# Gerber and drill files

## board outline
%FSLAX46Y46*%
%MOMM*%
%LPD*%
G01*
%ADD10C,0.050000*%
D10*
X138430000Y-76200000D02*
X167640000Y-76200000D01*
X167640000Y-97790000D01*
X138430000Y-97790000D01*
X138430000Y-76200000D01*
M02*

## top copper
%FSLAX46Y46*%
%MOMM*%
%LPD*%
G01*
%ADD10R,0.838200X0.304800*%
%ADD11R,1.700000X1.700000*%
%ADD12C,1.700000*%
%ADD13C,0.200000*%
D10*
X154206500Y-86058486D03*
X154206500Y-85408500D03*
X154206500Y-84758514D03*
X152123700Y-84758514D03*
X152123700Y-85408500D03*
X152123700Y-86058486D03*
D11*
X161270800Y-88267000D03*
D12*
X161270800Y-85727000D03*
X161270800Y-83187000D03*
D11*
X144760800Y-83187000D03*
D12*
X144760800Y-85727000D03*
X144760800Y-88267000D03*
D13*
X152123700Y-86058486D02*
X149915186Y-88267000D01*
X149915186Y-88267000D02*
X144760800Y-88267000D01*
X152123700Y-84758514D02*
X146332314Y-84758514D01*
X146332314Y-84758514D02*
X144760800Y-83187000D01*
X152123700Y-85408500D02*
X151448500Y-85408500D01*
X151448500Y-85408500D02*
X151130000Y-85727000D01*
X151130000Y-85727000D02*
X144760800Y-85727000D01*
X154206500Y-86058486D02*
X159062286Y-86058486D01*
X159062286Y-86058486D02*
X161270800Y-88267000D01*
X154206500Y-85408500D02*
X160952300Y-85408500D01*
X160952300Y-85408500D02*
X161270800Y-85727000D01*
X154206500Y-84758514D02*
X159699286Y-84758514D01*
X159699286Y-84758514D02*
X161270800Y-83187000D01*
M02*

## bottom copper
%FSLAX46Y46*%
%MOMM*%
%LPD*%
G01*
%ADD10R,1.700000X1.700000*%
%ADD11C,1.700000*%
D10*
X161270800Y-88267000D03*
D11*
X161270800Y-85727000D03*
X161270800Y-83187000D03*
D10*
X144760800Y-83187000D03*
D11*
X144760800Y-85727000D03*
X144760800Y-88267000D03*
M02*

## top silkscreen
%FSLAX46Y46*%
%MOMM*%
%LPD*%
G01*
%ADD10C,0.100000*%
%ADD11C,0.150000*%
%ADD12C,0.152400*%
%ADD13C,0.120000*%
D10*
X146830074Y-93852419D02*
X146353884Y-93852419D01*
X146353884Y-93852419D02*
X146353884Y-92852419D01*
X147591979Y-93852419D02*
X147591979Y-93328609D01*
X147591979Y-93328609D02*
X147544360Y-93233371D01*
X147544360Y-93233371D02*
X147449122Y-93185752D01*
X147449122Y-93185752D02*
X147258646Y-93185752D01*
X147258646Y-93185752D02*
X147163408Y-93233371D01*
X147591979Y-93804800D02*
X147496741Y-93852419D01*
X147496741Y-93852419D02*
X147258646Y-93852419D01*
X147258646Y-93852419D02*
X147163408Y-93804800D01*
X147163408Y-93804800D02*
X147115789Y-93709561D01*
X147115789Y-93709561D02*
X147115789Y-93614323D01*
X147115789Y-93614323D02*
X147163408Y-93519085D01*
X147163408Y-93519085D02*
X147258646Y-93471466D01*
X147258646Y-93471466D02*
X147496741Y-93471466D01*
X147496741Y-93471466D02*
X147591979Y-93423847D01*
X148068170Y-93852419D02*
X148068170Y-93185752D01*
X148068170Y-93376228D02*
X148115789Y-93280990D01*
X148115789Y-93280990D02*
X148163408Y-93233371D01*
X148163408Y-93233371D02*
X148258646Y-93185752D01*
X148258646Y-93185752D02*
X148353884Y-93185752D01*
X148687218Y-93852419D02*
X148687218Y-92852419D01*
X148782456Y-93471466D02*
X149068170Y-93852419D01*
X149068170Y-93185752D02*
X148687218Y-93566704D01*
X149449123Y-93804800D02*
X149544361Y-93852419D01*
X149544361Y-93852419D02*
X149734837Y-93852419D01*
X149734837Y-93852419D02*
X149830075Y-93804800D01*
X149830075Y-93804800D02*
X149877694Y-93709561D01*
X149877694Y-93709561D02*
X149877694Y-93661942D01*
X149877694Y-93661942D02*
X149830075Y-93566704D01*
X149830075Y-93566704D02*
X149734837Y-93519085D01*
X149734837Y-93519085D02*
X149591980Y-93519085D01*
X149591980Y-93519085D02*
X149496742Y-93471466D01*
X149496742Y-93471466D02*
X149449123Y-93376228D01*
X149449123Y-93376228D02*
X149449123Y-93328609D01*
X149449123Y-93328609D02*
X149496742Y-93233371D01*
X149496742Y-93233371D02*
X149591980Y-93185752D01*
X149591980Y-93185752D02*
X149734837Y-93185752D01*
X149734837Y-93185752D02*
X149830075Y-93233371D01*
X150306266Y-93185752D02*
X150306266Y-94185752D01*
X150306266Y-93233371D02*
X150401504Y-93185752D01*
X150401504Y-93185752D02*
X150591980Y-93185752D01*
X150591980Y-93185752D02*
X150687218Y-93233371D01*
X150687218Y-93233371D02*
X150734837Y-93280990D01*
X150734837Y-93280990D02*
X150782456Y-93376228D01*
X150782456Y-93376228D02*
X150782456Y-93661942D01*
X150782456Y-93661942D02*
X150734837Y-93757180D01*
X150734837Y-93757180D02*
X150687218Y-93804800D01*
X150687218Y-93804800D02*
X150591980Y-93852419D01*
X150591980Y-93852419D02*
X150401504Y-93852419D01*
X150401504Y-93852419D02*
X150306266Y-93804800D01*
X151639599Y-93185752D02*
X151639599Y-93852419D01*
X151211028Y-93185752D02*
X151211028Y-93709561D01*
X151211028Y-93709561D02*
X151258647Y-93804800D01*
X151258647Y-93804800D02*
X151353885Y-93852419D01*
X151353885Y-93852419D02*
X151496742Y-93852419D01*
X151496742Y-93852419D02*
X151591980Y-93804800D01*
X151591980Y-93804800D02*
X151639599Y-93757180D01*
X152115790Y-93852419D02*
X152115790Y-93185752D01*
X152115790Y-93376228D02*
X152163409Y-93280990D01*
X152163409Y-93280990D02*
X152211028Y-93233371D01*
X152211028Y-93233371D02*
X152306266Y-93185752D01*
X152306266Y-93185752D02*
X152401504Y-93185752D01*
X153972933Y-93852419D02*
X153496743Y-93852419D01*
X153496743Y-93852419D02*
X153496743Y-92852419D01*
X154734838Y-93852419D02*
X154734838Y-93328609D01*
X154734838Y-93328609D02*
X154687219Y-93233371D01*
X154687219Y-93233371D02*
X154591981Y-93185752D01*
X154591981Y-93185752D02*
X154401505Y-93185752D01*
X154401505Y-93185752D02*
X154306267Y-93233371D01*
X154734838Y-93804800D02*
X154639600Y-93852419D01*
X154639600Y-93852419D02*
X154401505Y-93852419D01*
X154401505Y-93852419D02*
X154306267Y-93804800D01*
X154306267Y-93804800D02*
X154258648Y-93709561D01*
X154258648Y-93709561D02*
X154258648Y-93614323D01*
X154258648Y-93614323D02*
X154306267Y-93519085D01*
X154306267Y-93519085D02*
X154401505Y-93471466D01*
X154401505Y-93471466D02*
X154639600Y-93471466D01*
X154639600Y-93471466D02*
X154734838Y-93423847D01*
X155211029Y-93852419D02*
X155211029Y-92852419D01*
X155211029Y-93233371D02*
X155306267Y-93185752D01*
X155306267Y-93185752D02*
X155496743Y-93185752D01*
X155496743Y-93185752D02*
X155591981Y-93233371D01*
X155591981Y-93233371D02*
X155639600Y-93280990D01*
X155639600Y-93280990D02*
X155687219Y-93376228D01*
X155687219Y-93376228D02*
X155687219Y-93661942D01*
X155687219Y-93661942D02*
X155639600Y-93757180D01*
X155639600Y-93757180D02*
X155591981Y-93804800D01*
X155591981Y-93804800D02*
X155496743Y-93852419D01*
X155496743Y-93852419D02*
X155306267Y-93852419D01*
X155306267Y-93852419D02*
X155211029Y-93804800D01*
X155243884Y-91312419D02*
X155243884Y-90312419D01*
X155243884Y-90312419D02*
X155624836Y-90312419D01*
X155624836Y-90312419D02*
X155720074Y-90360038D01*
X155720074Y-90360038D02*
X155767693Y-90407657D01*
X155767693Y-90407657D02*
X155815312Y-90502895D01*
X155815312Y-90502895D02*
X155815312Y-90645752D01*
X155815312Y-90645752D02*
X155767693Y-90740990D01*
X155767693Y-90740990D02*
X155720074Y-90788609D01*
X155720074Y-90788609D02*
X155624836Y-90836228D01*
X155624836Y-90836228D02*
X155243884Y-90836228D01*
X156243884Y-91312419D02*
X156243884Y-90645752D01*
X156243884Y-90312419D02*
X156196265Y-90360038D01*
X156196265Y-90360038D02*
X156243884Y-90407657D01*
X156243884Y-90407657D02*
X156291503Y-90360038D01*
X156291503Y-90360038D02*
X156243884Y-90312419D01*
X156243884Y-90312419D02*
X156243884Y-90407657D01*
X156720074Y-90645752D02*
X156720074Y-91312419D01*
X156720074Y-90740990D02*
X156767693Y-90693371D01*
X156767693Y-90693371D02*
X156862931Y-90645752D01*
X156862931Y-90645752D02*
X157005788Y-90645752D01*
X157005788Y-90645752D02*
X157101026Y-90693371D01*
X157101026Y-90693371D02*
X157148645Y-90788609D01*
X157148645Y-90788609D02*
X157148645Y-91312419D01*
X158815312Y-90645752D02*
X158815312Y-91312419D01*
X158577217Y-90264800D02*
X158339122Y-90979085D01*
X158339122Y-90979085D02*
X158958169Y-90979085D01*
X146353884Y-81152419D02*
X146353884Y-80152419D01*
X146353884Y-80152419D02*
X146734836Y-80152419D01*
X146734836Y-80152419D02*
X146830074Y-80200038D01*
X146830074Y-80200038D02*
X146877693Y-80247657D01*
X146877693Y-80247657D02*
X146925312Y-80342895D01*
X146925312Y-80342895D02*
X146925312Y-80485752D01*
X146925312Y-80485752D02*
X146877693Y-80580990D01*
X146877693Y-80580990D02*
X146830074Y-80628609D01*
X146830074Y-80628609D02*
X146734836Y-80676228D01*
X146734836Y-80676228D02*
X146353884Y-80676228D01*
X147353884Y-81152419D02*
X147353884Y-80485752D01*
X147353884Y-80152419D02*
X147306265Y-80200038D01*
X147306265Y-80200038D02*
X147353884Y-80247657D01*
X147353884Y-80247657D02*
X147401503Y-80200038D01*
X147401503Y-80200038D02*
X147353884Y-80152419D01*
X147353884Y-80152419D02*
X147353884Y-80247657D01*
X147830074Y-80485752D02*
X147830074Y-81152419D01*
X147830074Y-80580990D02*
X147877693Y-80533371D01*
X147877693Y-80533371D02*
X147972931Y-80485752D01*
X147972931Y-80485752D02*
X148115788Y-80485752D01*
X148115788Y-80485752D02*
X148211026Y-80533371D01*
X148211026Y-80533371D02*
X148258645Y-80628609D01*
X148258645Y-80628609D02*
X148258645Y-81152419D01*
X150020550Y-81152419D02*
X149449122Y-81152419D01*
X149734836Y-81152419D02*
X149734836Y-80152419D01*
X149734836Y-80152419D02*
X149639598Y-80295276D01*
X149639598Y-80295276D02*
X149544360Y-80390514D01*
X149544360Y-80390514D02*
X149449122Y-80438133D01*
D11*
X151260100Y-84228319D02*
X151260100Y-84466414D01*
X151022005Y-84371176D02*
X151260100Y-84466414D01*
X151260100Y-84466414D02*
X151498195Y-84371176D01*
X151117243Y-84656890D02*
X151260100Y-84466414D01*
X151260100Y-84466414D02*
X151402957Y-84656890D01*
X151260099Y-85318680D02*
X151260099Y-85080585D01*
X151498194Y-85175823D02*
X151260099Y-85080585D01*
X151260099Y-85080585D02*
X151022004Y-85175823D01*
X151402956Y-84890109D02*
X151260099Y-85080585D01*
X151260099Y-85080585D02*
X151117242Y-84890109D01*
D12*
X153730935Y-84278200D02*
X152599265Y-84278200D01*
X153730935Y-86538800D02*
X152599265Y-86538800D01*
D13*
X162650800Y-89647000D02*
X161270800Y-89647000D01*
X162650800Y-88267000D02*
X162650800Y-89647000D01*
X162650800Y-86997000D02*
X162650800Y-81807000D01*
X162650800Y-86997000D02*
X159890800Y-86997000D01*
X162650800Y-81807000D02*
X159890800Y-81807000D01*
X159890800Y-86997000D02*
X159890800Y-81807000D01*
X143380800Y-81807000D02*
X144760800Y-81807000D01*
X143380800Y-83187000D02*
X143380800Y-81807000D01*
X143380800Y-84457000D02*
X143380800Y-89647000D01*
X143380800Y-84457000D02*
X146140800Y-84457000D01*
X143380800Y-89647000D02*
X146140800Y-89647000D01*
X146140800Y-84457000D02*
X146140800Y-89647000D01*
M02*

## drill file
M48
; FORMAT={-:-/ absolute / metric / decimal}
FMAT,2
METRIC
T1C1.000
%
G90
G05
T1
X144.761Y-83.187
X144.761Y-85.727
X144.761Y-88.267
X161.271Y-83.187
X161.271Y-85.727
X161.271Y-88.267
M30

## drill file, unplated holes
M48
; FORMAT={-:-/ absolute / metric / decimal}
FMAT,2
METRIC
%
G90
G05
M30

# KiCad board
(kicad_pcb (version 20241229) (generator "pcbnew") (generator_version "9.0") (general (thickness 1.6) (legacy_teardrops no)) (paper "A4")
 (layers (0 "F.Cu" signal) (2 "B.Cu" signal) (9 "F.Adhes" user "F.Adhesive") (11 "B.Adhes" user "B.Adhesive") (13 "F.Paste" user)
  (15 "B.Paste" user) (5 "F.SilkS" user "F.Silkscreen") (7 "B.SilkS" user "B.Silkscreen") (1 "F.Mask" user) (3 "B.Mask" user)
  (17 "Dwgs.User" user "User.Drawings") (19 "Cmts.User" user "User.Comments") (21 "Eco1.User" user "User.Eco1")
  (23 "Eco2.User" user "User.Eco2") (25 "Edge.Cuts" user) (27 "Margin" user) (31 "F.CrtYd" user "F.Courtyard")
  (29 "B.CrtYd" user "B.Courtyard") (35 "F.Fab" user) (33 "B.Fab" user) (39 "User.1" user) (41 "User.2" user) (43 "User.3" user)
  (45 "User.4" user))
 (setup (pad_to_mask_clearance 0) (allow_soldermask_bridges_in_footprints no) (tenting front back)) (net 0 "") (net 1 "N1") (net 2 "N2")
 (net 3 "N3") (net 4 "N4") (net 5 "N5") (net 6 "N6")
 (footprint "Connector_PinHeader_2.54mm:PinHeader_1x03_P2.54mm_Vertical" (layer "F.Cu") (at 144.7608 83.187)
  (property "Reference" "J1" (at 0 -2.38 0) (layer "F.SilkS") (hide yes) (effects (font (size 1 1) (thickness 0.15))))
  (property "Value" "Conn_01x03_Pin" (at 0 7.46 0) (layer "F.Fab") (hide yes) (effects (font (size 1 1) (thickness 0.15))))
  (fp_line (start -1.38 -1.38) (end 0 -1.38) (stroke (width 0.12) (type solid)) (layer "F.SilkS"))
  (fp_line (start -1.38 0) (end -1.38 -1.38) (stroke (width 0.12) (type solid)) (layer "F.SilkS"))
  (fp_line (start -1.38 1.27) (end -1.38 6.46) (stroke (width 0.12) (type solid)) (layer "F.SilkS"))
  (fp_line (start -1.38 1.27) (end 1.38 1.27) (stroke (width 0.12) (type solid)) (layer "F.SilkS"))
  (fp_line (start -1.38 6.46) (end 1.38 6.46) (stroke (width 0.12) (type solid)) (layer "F.SilkS"))
  (fp_line (start 1.38 1.27) (end 1.38 6.46) (stroke (width 0.12) (type solid)) (layer "F.SilkS"))
  (pad "1" thru_hole rect (at 0 0) (size 1.7 1.7) (drill 1) (layers "*.Cu" "*.Mask") (remove_unused_layers no) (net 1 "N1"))
  (pad "2" thru_hole circle (at 0 2.54) (size 1.7 1.7) (drill 1) (layers "*.Cu" "*.Mask") (remove_unused_layers no) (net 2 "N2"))
  (pad "3" thru_hole circle (at 0 5.08) (size 1.7 1.7) (drill 1) (layers "*.Cu" "*.Mask") (remove_unused_layers no) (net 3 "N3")))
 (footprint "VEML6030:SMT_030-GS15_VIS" (layer "F.Cu") (at 153.1651 85.4085 180)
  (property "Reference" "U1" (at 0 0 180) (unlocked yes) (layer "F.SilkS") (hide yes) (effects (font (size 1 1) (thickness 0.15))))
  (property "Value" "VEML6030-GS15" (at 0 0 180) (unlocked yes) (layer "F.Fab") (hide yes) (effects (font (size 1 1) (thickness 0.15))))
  (fp_line (start -0.565835 1.1303) (end 0.565835 1.1303) (stroke (width 0.1524) (type solid)) (layer "F.SilkS"))
  (fp_line (start -0.565835 -1.1303) (end 0.565835 -1.1303) (stroke (width 0.1524) (type solid)) (layer "F.SilkS"))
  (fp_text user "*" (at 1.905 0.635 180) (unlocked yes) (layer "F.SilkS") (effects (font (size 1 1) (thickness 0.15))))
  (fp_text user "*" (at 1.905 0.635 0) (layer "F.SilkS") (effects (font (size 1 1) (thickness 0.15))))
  (pad "1" smd rect (at 1.0414 0.649986 180) (size 0.8382 0.3048) (layers "F.Cu" "F.Mask" "F.Paste") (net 1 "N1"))
  (pad "2" smd rect (at 1.0414 0 180) (size 0.8382 0.3048) (layers "F.Cu" "F.Mask" "F.Paste") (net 2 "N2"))
  (pad "3" smd rect (at 1.0414 -0.649986 180) (size 0.8382 0.3048) (layers "F.Cu" "F.Mask" "F.Paste") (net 3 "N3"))
  (pad "4" smd rect (at -1.0414 -0.649986 180) (size 0.8382 0.3048) (layers "F.Cu" "F.Mask" "F.Paste") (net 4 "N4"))
  (pad "5" smd rect (at -1.0414 0 180) (size 0.8382 0.3048) (layers "F.Cu" "F.Mask" "F.Paste") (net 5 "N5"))
  (pad "6" smd rect (at -1.0414 0.649986 180) (size 0.8382 0.3048) (layers "F.Cu" "F.Mask" "F.Paste") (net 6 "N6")))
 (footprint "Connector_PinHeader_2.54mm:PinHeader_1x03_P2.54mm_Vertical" (layer "F.Cu") (at 161.2708 88.267 180)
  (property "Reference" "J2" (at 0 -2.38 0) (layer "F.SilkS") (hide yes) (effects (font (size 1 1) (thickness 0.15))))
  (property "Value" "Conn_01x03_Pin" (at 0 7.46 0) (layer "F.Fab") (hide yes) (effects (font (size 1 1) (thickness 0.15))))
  (fp_line (start 1.38 1.27) (end 1.38 6.46) (stroke (width 0.12) (type solid)) (layer "F.SilkS"))
  (fp_line (start -1.38 6.46) (end 1.38 6.46) (stroke (width 0.12) (type solid)) (layer "F.SilkS"))
  (fp_line (start -1.38 1.27) (end 1.38 1.27) (stroke (width 0.12) (type solid)) (layer "F.SilkS"))
  (fp_line (start -1.38 1.27) (end -1.38 6.46) (stroke (width 0.12) (type solid)) (layer "F.SilkS"))
  (fp_line (start -1.38 0) (end -1.38 -1.38) (stroke (width 0.12) (type solid)) (layer "F.SilkS"))
  (fp_line (start -1.38 -1.38) (end 0 -1.38) (stroke (width 0.12) (type solid)) (layer "F.SilkS"))
  (pad "1" thru_hole rect (at 0 0 180) (size 1.7 1.7) (drill 1) (layers "*.Cu" "*.Mask") (remove_unused_layers no) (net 4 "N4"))
  (pad "2" thru_hole circle (at 0 2.54 180) (size 1.7 1.7) (drill 1) (layers "*.Cu" "*.Mask") (remove_unused_layers no) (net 5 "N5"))
  (pad "3" thru_hole circle (at 0 5.08 180) (size 1.7 1.7) (drill 1) (layers "*.Cu" "*.Mask") (remove_unused_layers no) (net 6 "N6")))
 (gr_rect (start 138.43 76.2) (end 167.64 97.79) (stroke (width 0.05) (type default)) (fill no) (layer "Edge.Cuts"))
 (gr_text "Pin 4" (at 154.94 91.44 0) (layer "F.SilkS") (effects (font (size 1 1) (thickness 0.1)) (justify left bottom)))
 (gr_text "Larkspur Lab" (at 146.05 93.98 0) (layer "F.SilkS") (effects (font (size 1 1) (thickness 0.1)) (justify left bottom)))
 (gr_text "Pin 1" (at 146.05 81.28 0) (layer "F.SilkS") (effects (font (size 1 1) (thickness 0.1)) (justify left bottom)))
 (segment (start 151.13 85.727) (end 144.7608 85.727) (width 0.2) (layer "F.Cu") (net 2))
 (segment (start 152.1237 85.4085) (end 151.4485 85.4085) (width 0.2) (layer "F.Cu") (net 2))
 (segment (start 151.4485 85.4085) (end 151.13 85.727) (width 0.2) (layer "F.Cu") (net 2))
 (segment (start 152.1237 84.758514) (end 146.332314 84.758514) (width 0.2) (layer "F.Cu") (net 1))
 (segment (start 146.332314 84.758514) (end 144.7608 83.187) (width 0.2) (layer "F.Cu") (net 1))
 (segment (start 152.1237 86.058486) (end 149.915186 88.267) (width 0.2) (layer "F.Cu") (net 3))
 (segment (start 149.915186 88.267) (end 144.7608 88.267) (width 0.2) (layer "F.Cu") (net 3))
 (segment (start 159.699286 84.758514) (end 161.2708 83.187) (width 0.2) (layer "F.Cu") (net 6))
 (segment (start 154.2065 84.758514) (end 159.699286 84.758514) (width 0.2) (layer "F.Cu") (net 6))
 (segment (start 154.2065 86.058486) (end 159.062286 86.058486) (width 0.2) (layer "F.Cu") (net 4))
 (segment (start 159.062286 86.058486) (end 161.2708 88.267) (width 0.2) (layer "F.Cu") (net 4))
 (segment (start 160.9523 85.4085) (end 161.2708 85.727) (width 0.2) (layer "F.Cu") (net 5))
 (segment (start 154.2065 85.4085) (end 160.9523 85.4085) (width 0.2) (layer "F.Cu") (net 5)))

